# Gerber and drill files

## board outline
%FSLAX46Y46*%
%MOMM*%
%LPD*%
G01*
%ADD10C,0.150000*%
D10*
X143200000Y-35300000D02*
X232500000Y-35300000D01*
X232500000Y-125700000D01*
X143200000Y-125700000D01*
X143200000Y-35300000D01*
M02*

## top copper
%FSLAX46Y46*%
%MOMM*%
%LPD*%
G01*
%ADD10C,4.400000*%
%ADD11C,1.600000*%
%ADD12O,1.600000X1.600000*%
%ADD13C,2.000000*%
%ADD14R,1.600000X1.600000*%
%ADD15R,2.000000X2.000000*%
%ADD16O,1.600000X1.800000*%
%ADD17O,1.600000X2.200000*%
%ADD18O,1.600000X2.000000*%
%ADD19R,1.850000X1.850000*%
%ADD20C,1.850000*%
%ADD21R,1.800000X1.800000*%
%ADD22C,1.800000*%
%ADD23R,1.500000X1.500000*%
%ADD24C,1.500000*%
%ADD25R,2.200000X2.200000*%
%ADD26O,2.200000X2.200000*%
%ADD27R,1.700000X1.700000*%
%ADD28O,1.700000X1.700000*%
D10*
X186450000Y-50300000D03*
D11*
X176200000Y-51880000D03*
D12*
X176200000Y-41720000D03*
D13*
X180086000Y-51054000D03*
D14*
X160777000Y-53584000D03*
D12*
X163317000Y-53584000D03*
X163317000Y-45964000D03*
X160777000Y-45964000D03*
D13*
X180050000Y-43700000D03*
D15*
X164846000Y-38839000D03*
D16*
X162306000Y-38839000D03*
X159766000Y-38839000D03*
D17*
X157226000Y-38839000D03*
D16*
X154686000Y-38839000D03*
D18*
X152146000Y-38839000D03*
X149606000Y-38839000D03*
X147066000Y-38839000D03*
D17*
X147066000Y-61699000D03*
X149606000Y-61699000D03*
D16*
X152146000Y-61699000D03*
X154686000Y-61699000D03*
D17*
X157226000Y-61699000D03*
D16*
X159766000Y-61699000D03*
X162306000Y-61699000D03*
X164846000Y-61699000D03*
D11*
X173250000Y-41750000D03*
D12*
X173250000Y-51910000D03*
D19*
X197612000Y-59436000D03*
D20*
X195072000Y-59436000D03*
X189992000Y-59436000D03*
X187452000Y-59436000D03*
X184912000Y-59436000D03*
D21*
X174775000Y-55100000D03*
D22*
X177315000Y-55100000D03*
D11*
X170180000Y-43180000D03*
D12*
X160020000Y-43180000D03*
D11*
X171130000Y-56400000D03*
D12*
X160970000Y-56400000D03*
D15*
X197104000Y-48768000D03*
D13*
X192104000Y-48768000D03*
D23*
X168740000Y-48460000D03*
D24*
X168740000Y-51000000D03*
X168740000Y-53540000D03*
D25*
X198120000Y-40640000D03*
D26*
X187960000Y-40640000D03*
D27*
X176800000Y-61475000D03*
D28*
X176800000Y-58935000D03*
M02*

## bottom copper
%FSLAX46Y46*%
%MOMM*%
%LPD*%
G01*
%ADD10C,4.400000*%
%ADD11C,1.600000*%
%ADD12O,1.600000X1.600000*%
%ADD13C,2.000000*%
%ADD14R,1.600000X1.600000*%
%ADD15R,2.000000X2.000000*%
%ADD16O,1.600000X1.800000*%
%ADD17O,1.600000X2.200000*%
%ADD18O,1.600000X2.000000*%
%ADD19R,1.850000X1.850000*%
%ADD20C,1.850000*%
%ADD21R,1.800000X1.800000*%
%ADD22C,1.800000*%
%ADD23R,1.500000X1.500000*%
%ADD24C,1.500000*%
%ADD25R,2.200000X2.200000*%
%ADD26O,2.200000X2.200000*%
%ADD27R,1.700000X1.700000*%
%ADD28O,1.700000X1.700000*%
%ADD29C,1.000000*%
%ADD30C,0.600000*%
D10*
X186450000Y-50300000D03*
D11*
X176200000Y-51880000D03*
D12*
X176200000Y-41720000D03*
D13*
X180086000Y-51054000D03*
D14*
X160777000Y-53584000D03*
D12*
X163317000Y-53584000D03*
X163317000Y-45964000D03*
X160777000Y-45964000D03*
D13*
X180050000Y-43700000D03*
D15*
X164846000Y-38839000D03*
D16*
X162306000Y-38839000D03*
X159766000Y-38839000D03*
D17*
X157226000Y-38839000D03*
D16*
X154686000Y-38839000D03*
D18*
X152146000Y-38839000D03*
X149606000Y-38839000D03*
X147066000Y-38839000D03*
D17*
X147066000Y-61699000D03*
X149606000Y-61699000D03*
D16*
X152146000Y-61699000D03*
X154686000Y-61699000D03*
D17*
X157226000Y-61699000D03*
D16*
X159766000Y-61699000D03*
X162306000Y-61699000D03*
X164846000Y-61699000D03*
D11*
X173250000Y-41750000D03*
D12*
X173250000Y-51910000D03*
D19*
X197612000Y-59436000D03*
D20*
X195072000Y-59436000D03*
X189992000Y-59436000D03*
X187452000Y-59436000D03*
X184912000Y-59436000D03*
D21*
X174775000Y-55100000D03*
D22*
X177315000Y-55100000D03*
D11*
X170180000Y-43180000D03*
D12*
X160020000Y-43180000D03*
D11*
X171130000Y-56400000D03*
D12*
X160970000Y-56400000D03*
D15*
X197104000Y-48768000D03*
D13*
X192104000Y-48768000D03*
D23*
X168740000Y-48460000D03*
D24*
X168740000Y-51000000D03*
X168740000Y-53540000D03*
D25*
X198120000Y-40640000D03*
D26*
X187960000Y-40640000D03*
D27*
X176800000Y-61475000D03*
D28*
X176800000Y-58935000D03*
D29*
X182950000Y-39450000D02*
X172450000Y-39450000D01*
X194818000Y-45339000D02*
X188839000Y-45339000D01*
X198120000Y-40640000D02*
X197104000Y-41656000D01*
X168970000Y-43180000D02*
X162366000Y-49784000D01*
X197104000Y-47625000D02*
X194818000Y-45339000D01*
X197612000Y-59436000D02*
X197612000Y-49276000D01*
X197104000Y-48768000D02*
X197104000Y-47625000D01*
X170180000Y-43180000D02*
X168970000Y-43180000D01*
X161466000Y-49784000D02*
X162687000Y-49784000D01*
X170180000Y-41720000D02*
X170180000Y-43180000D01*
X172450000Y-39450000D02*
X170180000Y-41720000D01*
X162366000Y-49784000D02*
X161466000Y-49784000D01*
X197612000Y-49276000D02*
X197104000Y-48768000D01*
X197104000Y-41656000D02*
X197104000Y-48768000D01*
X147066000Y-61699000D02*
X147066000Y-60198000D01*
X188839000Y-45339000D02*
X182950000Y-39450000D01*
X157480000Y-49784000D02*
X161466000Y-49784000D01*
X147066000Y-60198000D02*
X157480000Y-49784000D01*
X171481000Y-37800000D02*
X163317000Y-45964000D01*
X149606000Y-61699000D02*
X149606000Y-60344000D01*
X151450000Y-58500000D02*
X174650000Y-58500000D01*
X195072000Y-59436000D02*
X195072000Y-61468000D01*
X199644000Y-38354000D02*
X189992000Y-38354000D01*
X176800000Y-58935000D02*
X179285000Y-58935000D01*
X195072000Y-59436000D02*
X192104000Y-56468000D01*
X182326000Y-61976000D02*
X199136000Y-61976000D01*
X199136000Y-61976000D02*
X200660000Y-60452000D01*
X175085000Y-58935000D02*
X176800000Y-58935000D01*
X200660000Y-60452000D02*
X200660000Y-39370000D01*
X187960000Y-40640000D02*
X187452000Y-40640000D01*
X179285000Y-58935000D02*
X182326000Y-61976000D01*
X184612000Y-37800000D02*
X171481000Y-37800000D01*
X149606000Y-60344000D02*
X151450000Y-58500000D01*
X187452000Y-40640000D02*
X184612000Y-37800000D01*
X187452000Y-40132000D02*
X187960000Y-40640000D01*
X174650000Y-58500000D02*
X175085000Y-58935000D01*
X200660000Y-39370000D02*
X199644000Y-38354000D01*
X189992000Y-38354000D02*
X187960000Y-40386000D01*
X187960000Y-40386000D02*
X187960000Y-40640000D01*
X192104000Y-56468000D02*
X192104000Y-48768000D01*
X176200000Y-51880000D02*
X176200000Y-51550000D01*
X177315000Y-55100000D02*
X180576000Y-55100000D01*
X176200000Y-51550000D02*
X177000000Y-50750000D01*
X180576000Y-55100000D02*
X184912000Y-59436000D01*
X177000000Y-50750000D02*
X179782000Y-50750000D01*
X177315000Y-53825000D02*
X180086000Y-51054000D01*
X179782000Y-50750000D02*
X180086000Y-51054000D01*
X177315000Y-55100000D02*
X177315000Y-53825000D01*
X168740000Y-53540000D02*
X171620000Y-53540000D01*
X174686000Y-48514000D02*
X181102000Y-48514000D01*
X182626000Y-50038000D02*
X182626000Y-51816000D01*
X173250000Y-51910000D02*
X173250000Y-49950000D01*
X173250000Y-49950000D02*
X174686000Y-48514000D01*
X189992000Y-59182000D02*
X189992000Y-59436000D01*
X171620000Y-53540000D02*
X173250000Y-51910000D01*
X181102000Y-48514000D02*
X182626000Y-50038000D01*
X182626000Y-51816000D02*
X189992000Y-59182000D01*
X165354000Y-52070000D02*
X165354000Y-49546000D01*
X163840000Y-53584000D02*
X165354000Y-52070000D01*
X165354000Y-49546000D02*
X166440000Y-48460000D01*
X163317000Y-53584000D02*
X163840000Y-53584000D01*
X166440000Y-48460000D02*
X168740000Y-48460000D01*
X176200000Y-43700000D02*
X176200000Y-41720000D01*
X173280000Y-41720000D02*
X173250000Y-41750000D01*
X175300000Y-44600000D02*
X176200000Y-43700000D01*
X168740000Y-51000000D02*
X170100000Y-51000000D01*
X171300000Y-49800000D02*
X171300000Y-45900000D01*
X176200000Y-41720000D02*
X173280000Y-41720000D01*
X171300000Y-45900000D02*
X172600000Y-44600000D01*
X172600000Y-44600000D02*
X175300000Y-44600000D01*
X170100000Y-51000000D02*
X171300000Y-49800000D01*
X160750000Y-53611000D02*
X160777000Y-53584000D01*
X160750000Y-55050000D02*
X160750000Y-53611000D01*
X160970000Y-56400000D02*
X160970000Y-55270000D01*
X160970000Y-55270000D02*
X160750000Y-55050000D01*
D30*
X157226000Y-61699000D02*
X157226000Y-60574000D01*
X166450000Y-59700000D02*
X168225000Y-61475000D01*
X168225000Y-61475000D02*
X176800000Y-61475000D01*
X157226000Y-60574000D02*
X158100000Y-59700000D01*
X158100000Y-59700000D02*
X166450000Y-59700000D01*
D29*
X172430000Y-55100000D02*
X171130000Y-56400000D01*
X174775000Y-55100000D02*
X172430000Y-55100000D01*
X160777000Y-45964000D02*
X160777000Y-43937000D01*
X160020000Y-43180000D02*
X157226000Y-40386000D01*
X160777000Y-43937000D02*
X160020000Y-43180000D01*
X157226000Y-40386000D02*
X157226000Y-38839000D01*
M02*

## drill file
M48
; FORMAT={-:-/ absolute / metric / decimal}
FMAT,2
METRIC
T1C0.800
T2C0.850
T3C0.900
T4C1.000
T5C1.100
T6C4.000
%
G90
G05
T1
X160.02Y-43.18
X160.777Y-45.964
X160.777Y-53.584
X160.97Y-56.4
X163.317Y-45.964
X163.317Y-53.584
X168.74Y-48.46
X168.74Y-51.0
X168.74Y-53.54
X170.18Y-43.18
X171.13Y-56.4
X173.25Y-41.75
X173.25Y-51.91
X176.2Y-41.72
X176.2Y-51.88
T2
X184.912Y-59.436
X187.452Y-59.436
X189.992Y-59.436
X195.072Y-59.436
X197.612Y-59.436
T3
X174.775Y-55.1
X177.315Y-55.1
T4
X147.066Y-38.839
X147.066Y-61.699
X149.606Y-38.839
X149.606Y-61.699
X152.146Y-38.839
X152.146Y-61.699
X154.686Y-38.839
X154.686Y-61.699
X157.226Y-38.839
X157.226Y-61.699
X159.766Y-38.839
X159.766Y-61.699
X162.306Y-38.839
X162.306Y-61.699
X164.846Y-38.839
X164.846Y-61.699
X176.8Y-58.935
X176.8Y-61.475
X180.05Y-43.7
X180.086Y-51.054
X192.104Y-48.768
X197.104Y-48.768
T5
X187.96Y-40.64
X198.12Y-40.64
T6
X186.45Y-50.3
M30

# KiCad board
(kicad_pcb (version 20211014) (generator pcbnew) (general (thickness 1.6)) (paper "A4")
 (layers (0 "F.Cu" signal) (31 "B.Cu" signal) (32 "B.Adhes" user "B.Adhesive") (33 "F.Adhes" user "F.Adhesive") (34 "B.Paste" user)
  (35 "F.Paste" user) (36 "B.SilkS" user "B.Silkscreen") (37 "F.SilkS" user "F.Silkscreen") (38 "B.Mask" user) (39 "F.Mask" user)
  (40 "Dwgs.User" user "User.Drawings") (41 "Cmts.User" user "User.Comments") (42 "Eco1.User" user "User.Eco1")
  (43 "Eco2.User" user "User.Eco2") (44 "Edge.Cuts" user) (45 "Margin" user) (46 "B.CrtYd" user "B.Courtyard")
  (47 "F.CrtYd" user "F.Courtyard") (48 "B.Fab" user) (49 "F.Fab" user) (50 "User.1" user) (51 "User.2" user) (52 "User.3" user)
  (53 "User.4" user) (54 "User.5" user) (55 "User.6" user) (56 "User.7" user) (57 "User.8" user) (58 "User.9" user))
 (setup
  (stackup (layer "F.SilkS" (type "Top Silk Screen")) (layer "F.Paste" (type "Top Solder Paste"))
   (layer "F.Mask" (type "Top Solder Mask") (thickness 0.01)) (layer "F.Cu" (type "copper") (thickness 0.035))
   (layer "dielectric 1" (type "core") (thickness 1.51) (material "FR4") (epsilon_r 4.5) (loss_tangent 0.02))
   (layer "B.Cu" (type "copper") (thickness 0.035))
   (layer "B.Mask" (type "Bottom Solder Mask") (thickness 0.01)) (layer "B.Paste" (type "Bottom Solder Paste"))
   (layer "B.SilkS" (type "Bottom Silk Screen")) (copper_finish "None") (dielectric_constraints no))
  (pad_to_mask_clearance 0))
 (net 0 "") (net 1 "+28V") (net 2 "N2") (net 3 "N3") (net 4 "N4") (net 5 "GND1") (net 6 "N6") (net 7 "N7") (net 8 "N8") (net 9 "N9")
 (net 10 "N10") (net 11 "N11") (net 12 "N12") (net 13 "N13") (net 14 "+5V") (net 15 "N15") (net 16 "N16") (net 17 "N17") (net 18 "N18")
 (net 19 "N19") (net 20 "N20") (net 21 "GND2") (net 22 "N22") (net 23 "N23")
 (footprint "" (layer "F.Cu") (at 186.45 50.3)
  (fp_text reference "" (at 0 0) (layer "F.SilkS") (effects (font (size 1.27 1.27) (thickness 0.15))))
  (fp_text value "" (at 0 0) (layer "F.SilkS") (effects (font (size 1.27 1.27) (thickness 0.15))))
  (pad "1" thru_hole circle (at 0 0) (size 4.4 4.4) (drill 4) (layers *.Cu *.Mask)))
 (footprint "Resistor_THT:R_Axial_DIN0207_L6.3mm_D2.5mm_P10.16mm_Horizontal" (layer "F.Cu") (at 176.2 51.88 90)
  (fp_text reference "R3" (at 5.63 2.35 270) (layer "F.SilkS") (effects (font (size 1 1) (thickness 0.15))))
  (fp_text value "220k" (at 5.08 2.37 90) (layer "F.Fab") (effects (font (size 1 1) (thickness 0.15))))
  (pad "1" thru_hole circle (at 0 0 90) (size 1.6 1.6) (drill 0.8) (layers *.Cu *.Mask) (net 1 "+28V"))
  (pad "2" thru_hole oval (at 10.16 0 90) (size 1.6 1.6) (drill 0.8) (layers *.Cu *.Mask) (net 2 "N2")))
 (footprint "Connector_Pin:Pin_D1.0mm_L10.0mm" (layer "F.Cu") (at 180.086 51.054)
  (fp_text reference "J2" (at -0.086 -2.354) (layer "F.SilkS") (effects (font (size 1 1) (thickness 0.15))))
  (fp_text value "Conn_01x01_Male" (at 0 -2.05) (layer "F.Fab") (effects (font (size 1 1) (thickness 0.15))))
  (pad "1" thru_hole circle (at 0 0) (size 2 2) (drill 1) (layers *.Cu *.Mask) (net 1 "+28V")))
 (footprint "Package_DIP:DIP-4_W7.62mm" (layer "F.Cu") (at 160.777 53.584 90)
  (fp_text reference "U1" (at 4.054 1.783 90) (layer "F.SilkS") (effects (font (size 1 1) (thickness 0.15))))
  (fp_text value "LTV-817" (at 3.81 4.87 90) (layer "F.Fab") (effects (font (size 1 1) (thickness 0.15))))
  (pad "1" thru_hole rect (at 0 0 90) (size 1.6 1.6) (drill 0.8) (layers *.Cu *.Mask) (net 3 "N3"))
  (pad "2" thru_hole oval (at 0 2.54 90) (size 1.6 1.6) (drill 0.8) (layers *.Cu *.Mask) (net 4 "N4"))
  (pad "3" thru_hole oval (at 7.62 2.54 90) (size 1.6 1.6) (drill 0.8) (layers *.Cu *.Mask) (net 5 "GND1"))
  (pad "4" thru_hole oval (at 7.62 0 90) (size 1.6 1.6) (drill 0.8) (layers *.Cu *.Mask) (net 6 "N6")))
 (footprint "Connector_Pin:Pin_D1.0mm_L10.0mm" (layer "F.Cu") (at 180.05 43.7)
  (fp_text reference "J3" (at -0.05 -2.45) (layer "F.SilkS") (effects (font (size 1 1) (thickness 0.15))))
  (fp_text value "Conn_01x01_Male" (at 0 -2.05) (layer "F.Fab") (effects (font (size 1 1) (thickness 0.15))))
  (pad "1" thru_hole circle (at 0 0) (size 2 2) (drill 1) (layers *.Cu *.Mask) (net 2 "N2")))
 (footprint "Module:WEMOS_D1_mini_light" (layer "F.Cu") (at 164.846 38.839 -90)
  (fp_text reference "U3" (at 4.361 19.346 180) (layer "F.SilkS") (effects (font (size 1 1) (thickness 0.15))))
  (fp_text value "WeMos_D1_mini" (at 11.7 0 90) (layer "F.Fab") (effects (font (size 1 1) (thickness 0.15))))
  (pad "1" thru_hole rect (at 0 0 270) (size 2 2) (drill 1) (layers *.Cu *.Mask) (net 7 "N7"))
  (pad "2" thru_hole oval (at 0 2.54 270) (size 1.8 1.6) (drill 1) (layers *.Cu *.Mask) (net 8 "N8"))
  (pad "3" thru_hole oval (at 0 5.08 270) (size 1.8 1.6) (drill 1) (layers *.Cu *.Mask) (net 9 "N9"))
  (pad "4" thru_hole oval (at 0 7.62 270) (size 2.2 1.6) (drill 1) (layers *.Cu *.Mask) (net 6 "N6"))
  (pad "5" thru_hole oval (at 0 10.16 270) (size 1.8 1.6) (drill 1) (layers *.Cu *.Mask) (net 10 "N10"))
  (pad "6" thru_hole oval (at 0 12.7 270) (size 2 1.6) (drill 1) (layers *.Cu *.Mask) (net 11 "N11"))
  (pad "7" thru_hole oval (at 0 15.24 270) (size 2 1.6) (drill 1) (layers *.Cu *.Mask) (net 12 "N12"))
  (pad "8" thru_hole oval (at 0 17.78 270) (size 2 1.6) (drill 1) (layers *.Cu *.Mask) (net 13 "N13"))
  (pad "9" thru_hole oval (at 22.86 17.78 270) (size 2.2 1.6) (drill 1) (layers *.Cu *.Mask) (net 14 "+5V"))
  (pad "10" thru_hole oval (at 22.86 15.24 270) (size 2.2 1.6) (drill 1) (layers *.Cu *.Mask) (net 5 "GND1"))
  (pad "11" thru_hole oval (at 22.86 12.7 270) (size 1.8 1.6) (drill 1) (layers *.Cu *.Mask) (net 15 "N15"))
  (pad "12" thru_hole oval (at 22.86 10.16 270) (size 1.8 1.6) (drill 1) (layers *.Cu *.Mask) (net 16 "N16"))
  (pad "13" thru_hole oval (at 22.86 7.62 270) (size 2.2 1.6) (drill 1) (layers *.Cu *.Mask) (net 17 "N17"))
  (pad "14" thru_hole oval (at 22.86 5.08 270) (size 1.8 1.6) (drill 1) (layers *.Cu *.Mask) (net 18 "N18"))
  (pad "15" thru_hole oval (at 22.86 2.54 270) (size 1.8 1.6) (drill 1) (layers *.Cu *.Mask) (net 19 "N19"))
  (pad "16" thru_hole oval (at 22.86 0 270) (size 1.8 1.6) (drill 1) (layers *.Cu *.Mask) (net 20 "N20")))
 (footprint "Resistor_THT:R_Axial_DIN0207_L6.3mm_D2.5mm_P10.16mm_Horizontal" (layer "F.Cu") (at 173.25 41.75 -90)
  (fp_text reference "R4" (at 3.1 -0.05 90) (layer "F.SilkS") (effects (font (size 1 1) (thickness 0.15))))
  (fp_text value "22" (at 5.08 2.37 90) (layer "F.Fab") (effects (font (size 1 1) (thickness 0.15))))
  (pad "1" thru_hole circle (at 0 0 270) (size 1.6 1.6) (drill 0.8) (layers *.Cu *.Mask) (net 2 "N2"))
  (pad "2" thru_hole oval (at 10.16 0 270) (size 1.6 1.6) (drill 0.8) (layers *.Cu *.Mask) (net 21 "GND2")))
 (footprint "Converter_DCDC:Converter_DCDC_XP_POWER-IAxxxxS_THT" (layer "F.Cu") (at 197.612 59.436 -90)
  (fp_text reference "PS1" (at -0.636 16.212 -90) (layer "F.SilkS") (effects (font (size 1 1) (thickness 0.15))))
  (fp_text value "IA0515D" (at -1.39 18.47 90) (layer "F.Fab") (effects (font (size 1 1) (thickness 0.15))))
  (pad "1" thru_hole rect (at 0 0 270) (size 1.85 1.85) (drill 0.85) (layers *.Cu *.Mask) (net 14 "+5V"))
  (pad "2" thru_hole circle (at 0 2.54 270) (size 1.85 1.85) (drill 0.85) (layers *.Cu *.Mask) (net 5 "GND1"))
  (pad "4" thru_hole circle (at 0 7.62 270) (size 1.85 1.85) (drill 0.85) (layers *.Cu *.Mask) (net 21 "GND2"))
  (pad "5" thru_hole circle (at 0 10.16 270) (size 1.85 1.85) (drill 0.85) (layers *.Cu *.Mask) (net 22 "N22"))
  (pad "6" thru_hole circle (at 0 12.7 270) (size 1.85 1.85) (drill 0.85) (layers *.Cu *.Mask) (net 1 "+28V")))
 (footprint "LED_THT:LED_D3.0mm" (layer "F.Cu") (at 174.775 55.1)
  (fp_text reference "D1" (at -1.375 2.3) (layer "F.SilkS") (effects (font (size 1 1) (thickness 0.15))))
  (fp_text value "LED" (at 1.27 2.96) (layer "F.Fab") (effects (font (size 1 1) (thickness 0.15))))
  (pad "1" thru_hole rect (at 0 0) (size 1.8 1.8) (drill 0.9) (layers *.Cu *.Mask) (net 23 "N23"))
  (pad "2" thru_hole circle (at 2.54 0) (size 1.8 1.8) (drill 0.9) (layers *.Cu *.Mask) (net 1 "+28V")))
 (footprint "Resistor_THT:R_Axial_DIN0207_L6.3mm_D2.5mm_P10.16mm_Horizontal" (layer "F.Cu") (at 170.18 43.18 180)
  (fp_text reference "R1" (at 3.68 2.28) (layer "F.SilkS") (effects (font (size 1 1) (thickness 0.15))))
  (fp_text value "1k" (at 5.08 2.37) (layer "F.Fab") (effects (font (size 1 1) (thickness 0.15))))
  (pad "1" thru_hole circle (at 0 0 180) (size 1.6 1.6) (drill 0.8) (layers *.Cu *.Mask) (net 14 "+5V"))
  (pad "2" thru_hole oval (at 10.16 0 180) (size 1.6 1.6) (drill 0.8) (layers *.Cu *.Mask) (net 6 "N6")))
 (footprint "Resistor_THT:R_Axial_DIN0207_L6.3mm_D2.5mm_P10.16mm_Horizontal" (layer "F.Cu") (at 171.13 56.4 180)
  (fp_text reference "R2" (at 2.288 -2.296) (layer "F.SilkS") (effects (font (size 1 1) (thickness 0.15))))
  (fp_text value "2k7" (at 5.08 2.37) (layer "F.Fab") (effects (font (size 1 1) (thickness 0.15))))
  (pad "1" thru_hole circle (at 0 0 180) (size 1.6 1.6) (drill 0.8) (layers *.Cu *.Mask) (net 23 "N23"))
  (pad "2" thru_hole oval (at 10.16 0 180) (size 1.6 1.6) (drill 0.8) (layers *.Cu *.Mask) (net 3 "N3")))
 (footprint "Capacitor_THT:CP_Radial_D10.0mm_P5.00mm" (layer "F.Cu") (at 197.104 48.768 180)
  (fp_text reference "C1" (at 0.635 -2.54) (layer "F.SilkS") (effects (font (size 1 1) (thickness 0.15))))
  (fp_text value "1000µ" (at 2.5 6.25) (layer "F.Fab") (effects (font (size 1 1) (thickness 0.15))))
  (pad "1" thru_hole rect (at 0 0 180) (size 2 2) (drill 1) (layers *.Cu *.Mask) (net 14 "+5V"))
  (pad "2" thru_hole circle (at 5 0 180) (size 2 2) (drill 1) (layers *.Cu *.Mask) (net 5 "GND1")))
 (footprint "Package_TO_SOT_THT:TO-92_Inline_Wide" (layer "F.Cu") (at 168.74 48.46 -90)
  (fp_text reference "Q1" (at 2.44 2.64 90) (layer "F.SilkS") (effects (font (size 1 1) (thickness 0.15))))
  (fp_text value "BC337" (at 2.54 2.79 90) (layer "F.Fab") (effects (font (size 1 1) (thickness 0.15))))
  (pad "1" thru_hole rect (at 0 0 270) (size 1.5 1.5) (drill 0.8) (layers *.Cu *.Mask) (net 4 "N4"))
  (pad "2" thru_hole circle (at 2.54 0 270) (size 1.5 1.5) (drill 0.8) (layers *.Cu *.Mask) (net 2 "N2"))
  (pad "3" thru_hole circle (at 5.08 0 270) (size 1.5 1.5) (drill 0.8) (layers *.Cu *.Mask) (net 21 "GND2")))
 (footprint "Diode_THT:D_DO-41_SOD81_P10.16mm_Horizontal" (layer "F.Cu") (at 198.12 40.64 180)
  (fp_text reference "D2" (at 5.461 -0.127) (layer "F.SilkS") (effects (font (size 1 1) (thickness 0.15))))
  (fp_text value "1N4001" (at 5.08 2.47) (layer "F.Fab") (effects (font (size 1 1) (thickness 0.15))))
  (pad "1" thru_hole rect (at 0 0 180) (size 2.2 2.2) (drill 1.1) (layers *.Cu *.Mask) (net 14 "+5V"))
  (pad "2" thru_hole oval (at 10.16 0 180) (size 2.2 2.2) (drill 1.1) (layers *.Cu *.Mask) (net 5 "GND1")))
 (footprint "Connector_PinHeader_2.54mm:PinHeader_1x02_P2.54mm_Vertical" (layer "F.Cu") (at 176.8 61.475 180)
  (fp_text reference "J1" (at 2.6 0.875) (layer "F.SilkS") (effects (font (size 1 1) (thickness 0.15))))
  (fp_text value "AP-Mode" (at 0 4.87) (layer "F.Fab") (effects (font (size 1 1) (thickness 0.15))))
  (pad "1" thru_hole rect (at 0 0 180) (size 1.7 1.7) (drill 1) (layers *.Cu *.Mask) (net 17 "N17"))
  (pad "2" thru_hole oval (at 0 2.54 180) (size 1.7 1.7) (drill 1) (layers *.Cu *.Mask) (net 5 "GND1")))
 (gr_rect (start 143.2 35.3) (end 232.5 125.7) (layer "Edge.Cuts") (width 0.15) (fill none))
 (segment (start 182.95 39.45) (end 172.45 39.45) (width 1) (layer "B.Cu") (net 14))
 (segment (start 194.818 45.339) (end 188.839 45.339) (width 1) (layer "B.Cu") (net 14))
 (segment (start 198.12 40.64) (end 197.104 41.656) (width 1) (layer "B.Cu") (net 14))
 (segment (start 168.97 43.18) (end 162.366 49.784) (width 1) (layer "B.Cu") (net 14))
 (segment (start 197.104 47.625) (end 194.818 45.339) (width 1) (layer "B.Cu") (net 14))
 (segment (start 197.612 59.436) (end 197.612 49.276) (width 1) (layer "B.Cu") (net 14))
 (segment (start 197.104 48.768) (end 197.104 47.625) (width 1) (layer "B.Cu") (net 14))
 (segment (start 170.18 43.18) (end 168.97 43.18) (width 1) (layer "B.Cu") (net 14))
 (segment (start 161.466 49.784) (end 162.687 49.784) (width 1) (layer "B.Cu") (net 14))
 (segment (start 170.18 41.72) (end 170.18 43.18) (width 1) (layer "B.Cu") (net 14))
 (segment (start 172.45 39.45) (end 170.18 41.72) (width 1) (layer "B.Cu") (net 14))
 (segment (start 162.366 49.784) (end 161.466 49.784) (width 1) (layer "B.Cu") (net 14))
 (segment (start 197.612 49.276) (end 197.104 48.768) (width 1) (layer "B.Cu") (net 14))
 (segment (start 197.104 41.656) (end 197.104 48.768) (width 1) (layer "B.Cu") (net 14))
 (segment (start 147.066 61.699) (end 147.066 60.198) (width 1) (layer "B.Cu") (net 14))
 (segment (start 188.839 45.339) (end 182.95 39.45) (width 1) (layer "B.Cu") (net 14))
 (segment (start 157.48 49.784) (end 161.466 49.784) (width 1) (layer "B.Cu") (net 14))
 (segment (start 147.066 60.198) (end 157.48 49.784) (width 1) (layer "B.Cu") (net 14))
 (segment (start 171.481 37.8) (end 163.317 45.964) (width 1) (layer "B.Cu") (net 5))
 (segment (start 149.606 61.699) (end 149.606 60.344) (width 1) (layer "B.Cu") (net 5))
 (segment (start 151.45 58.5) (end 174.65 58.5) (width 1) (layer "B.Cu") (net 5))
 (segment (start 195.072 59.436) (end 195.072 61.468) (width 1) (layer "B.Cu") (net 5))
 (segment (start 199.644 38.354) (end 189.992 38.354) (width 1) (layer "B.Cu") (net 5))
 (segment (start 176.8 58.935) (end 179.285 58.935) (width 1) (layer "B.Cu") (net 5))
 (segment (start 195.072 59.436) (end 192.104 56.468) (width 1) (layer "B.Cu") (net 5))
 (segment (start 182.326 61.976) (end 199.136 61.976) (width 1) (layer "B.Cu") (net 5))
 (segment (start 199.136 61.976) (end 200.66 60.452) (width 1) (layer "B.Cu") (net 5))
 (segment (start 175.085 58.935) (end 176.8 58.935) (width 1) (layer "B.Cu") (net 5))
 (segment (start 200.66 60.452) (end 200.66 39.37) (width 1) (layer "B.Cu") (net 5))
 (segment (start 187.96 40.64) (end 187.452 40.64) (width 1) (layer "B.Cu") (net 5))
 (segment (start 179.285 58.935) (end 182.326 61.976) (width 1) (layer "B.Cu") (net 5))
 (segment (start 184.612 37.8) (end 171.481 37.8) (width 1) (layer "B.Cu") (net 5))
 (segment (start 149.606 60.344) (end 151.45 58.5) (width 1) (layer "B.Cu") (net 5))
 (segment (start 187.452 40.64) (end 184.612 37.8) (width 1) (layer "B.Cu") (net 5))
 (segment (start 187.452 40.132) (end 187.96 40.64) (width 1) (layer "B.Cu") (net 5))
 (segment (start 174.65 58.5) (end 175.085 58.935) (width 1) (layer "B.Cu") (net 5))
 (segment (start 200.66 39.37) (end 199.644 38.354) (width 1) (layer "B.Cu") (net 5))
 (segment (start 189.992 38.354) (end 187.96 40.386) (width 1) (layer "B.Cu") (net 5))
 (segment (start 187.96 40.386) (end 187.96 40.64) (width 1) (layer "B.Cu") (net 5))
 (segment (start 192.104 56.468) (end 192.104 48.768) (width 1) (layer "B.Cu") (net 5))
 (segment (start 176.2 51.88) (end 176.2 51.55) (width 1) (layer "B.Cu") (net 1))
 (segment (start 177.315 55.1) (end 180.576 55.1) (width 1) (layer "B.Cu") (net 1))
 (segment (start 176.2 51.55) (end 177 50.75) (width 1) (layer "B.Cu") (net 1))
 (segment (start 180.576 55.1) (end 184.912 59.436) (width 1) (layer "B.Cu") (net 1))
 (segment (start 177 50.75) (end 179.782 50.75) (width 1) (layer "B.Cu") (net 1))
 (segment (start 177.315 53.825) (end 180.086 51.054) (width 1) (layer "B.Cu") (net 1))
 (segment (start 179.782 50.75) (end 180.086 51.054) (width 1) (layer "B.Cu") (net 1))
 (segment (start 177.315 55.1) (end 177.315 53.825) (width 1) (layer "B.Cu") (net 1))
 (segment (start 168.74 53.54) (end 171.62 53.54) (width 1) (layer "B.Cu") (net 21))
 (segment (start 174.686 48.514) (end 181.102 48.514) (width 1) (layer "B.Cu") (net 21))
 (segment (start 182.626 50.038) (end 182.626 51.816) (width 1) (layer "B.Cu") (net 21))
 (segment (start 173.25 51.91) (end 173.25 49.95) (width 1) (layer "B.Cu") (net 21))
 (segment (start 173.25 49.95) (end 174.686 48.514) (width 1) (layer "B.Cu") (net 21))
 (segment (start 189.992 59.182) (end 189.992 59.436) (width 1) (layer "B.Cu") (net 21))
 (segment (start 171.62 53.54) (end 173.25 51.91) (width 1) (layer "B.Cu") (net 21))
 (segment (start 181.102 48.514) (end 182.626 50.038) (width 1) (layer "B.Cu") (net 21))
 (segment (start 182.626 51.816) (end 189.992 59.182) (width 1) (layer "B.Cu") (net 21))
 (segment (start 165.354 52.07) (end 165.354 49.546) (width 1) (layer "B.Cu") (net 4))
 (segment (start 163.84 53.584) (end 165.354 52.07) (width 1) (layer "B.Cu") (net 4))
 (segment (start 165.354 49.546) (end 166.44 48.46) (width 1) (layer "B.Cu") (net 4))
 (segment (start 163.317 53.584) (end 163.84 53.584) (width 1) (layer "B.Cu") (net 4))
 (segment (start 166.44 48.46) (end 168.74 48.46) (width 1) (layer "B.Cu") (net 4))
 (segment (start 176.2 43.7) (end 176.2 41.72) (width 1) (layer "B.Cu") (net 2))
 (segment (start 173.28 41.72) (end 173.25 41.75) (width 1) (layer "B.Cu") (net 2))
 (segment (start 175.3 44.6) (end 176.2 43.7) (width 1) (layer "B.Cu") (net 2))
 (segment (start 168.74 51) (end 170.1 51) (width 1) (layer "B.Cu") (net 2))
 (segment (start 171.3 49.8) (end 171.3 45.9) (width 1) (layer "B.Cu") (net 2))
 (segment (start 176.2 41.72) (end 173.28 41.72) (width 1) (layer "B.Cu") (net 2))
 (segment (start 171.3 45.9) (end 172.6 44.6) (width 1) (layer "B.Cu") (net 2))
 (segment (start 172.6 44.6) (end 175.3 44.6) (width 1) (layer "B.Cu") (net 2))
 (segment (start 170.1 51) (end 171.3 49.8) (width 1) (layer "B.Cu") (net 2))
 (segment (start 160.75 53.611) (end 160.777 53.584) (width 1) (layer "B.Cu") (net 3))
 (segment (start 160.75 55.05) (end 160.75 53.611) (width 1) (layer "B.Cu") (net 3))
 (segment (start 160.97 56.4) (end 160.97 55.27) (width 1) (layer "B.Cu") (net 3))
 (segment (start 160.97 55.27) (end 160.75 55.05) (width 1) (layer "B.Cu") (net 3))
 (segment (start 157.226 61.699) (end 157.226 60.574) (width 0.6) (layer "B.Cu") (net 17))
 (segment (start 166.45 59.7) (end 168.225 61.475) (width 0.6) (layer "B.Cu") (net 17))
 (segment (start 168.225 61.475) (end 176.8 61.475) (width 0.6) (layer "B.Cu") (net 17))
 (segment (start 157.226 60.574) (end 158.1 59.7) (width 0.6) (layer "B.Cu") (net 17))
 (segment (start 158.1 59.7) (end 166.45 59.7) (width 0.6) (layer "B.Cu") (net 17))
 (segment (start 172.43 55.1) (end 171.13 56.4) (width 1) (layer "B.Cu") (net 23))
 (segment (start 174.775 55.1) (end 172.43 55.1) (width 1) (layer "B.Cu") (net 23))
 (segment (start 160.777 45.964) (end 160.777 43.937) (width 1) (layer "B.Cu") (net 6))
 (segment (start 160.02 43.18) (end 157.226 40.386) (width 1) (layer "B.Cu") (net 6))
 (segment (start 160.777 43.937) (end 160.02 43.18) (width 1) (layer "B.Cu") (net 6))
 (segment (start 157.226 40.386) (end 157.226 38.839) (width 1) (layer "B.Cu") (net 6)))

